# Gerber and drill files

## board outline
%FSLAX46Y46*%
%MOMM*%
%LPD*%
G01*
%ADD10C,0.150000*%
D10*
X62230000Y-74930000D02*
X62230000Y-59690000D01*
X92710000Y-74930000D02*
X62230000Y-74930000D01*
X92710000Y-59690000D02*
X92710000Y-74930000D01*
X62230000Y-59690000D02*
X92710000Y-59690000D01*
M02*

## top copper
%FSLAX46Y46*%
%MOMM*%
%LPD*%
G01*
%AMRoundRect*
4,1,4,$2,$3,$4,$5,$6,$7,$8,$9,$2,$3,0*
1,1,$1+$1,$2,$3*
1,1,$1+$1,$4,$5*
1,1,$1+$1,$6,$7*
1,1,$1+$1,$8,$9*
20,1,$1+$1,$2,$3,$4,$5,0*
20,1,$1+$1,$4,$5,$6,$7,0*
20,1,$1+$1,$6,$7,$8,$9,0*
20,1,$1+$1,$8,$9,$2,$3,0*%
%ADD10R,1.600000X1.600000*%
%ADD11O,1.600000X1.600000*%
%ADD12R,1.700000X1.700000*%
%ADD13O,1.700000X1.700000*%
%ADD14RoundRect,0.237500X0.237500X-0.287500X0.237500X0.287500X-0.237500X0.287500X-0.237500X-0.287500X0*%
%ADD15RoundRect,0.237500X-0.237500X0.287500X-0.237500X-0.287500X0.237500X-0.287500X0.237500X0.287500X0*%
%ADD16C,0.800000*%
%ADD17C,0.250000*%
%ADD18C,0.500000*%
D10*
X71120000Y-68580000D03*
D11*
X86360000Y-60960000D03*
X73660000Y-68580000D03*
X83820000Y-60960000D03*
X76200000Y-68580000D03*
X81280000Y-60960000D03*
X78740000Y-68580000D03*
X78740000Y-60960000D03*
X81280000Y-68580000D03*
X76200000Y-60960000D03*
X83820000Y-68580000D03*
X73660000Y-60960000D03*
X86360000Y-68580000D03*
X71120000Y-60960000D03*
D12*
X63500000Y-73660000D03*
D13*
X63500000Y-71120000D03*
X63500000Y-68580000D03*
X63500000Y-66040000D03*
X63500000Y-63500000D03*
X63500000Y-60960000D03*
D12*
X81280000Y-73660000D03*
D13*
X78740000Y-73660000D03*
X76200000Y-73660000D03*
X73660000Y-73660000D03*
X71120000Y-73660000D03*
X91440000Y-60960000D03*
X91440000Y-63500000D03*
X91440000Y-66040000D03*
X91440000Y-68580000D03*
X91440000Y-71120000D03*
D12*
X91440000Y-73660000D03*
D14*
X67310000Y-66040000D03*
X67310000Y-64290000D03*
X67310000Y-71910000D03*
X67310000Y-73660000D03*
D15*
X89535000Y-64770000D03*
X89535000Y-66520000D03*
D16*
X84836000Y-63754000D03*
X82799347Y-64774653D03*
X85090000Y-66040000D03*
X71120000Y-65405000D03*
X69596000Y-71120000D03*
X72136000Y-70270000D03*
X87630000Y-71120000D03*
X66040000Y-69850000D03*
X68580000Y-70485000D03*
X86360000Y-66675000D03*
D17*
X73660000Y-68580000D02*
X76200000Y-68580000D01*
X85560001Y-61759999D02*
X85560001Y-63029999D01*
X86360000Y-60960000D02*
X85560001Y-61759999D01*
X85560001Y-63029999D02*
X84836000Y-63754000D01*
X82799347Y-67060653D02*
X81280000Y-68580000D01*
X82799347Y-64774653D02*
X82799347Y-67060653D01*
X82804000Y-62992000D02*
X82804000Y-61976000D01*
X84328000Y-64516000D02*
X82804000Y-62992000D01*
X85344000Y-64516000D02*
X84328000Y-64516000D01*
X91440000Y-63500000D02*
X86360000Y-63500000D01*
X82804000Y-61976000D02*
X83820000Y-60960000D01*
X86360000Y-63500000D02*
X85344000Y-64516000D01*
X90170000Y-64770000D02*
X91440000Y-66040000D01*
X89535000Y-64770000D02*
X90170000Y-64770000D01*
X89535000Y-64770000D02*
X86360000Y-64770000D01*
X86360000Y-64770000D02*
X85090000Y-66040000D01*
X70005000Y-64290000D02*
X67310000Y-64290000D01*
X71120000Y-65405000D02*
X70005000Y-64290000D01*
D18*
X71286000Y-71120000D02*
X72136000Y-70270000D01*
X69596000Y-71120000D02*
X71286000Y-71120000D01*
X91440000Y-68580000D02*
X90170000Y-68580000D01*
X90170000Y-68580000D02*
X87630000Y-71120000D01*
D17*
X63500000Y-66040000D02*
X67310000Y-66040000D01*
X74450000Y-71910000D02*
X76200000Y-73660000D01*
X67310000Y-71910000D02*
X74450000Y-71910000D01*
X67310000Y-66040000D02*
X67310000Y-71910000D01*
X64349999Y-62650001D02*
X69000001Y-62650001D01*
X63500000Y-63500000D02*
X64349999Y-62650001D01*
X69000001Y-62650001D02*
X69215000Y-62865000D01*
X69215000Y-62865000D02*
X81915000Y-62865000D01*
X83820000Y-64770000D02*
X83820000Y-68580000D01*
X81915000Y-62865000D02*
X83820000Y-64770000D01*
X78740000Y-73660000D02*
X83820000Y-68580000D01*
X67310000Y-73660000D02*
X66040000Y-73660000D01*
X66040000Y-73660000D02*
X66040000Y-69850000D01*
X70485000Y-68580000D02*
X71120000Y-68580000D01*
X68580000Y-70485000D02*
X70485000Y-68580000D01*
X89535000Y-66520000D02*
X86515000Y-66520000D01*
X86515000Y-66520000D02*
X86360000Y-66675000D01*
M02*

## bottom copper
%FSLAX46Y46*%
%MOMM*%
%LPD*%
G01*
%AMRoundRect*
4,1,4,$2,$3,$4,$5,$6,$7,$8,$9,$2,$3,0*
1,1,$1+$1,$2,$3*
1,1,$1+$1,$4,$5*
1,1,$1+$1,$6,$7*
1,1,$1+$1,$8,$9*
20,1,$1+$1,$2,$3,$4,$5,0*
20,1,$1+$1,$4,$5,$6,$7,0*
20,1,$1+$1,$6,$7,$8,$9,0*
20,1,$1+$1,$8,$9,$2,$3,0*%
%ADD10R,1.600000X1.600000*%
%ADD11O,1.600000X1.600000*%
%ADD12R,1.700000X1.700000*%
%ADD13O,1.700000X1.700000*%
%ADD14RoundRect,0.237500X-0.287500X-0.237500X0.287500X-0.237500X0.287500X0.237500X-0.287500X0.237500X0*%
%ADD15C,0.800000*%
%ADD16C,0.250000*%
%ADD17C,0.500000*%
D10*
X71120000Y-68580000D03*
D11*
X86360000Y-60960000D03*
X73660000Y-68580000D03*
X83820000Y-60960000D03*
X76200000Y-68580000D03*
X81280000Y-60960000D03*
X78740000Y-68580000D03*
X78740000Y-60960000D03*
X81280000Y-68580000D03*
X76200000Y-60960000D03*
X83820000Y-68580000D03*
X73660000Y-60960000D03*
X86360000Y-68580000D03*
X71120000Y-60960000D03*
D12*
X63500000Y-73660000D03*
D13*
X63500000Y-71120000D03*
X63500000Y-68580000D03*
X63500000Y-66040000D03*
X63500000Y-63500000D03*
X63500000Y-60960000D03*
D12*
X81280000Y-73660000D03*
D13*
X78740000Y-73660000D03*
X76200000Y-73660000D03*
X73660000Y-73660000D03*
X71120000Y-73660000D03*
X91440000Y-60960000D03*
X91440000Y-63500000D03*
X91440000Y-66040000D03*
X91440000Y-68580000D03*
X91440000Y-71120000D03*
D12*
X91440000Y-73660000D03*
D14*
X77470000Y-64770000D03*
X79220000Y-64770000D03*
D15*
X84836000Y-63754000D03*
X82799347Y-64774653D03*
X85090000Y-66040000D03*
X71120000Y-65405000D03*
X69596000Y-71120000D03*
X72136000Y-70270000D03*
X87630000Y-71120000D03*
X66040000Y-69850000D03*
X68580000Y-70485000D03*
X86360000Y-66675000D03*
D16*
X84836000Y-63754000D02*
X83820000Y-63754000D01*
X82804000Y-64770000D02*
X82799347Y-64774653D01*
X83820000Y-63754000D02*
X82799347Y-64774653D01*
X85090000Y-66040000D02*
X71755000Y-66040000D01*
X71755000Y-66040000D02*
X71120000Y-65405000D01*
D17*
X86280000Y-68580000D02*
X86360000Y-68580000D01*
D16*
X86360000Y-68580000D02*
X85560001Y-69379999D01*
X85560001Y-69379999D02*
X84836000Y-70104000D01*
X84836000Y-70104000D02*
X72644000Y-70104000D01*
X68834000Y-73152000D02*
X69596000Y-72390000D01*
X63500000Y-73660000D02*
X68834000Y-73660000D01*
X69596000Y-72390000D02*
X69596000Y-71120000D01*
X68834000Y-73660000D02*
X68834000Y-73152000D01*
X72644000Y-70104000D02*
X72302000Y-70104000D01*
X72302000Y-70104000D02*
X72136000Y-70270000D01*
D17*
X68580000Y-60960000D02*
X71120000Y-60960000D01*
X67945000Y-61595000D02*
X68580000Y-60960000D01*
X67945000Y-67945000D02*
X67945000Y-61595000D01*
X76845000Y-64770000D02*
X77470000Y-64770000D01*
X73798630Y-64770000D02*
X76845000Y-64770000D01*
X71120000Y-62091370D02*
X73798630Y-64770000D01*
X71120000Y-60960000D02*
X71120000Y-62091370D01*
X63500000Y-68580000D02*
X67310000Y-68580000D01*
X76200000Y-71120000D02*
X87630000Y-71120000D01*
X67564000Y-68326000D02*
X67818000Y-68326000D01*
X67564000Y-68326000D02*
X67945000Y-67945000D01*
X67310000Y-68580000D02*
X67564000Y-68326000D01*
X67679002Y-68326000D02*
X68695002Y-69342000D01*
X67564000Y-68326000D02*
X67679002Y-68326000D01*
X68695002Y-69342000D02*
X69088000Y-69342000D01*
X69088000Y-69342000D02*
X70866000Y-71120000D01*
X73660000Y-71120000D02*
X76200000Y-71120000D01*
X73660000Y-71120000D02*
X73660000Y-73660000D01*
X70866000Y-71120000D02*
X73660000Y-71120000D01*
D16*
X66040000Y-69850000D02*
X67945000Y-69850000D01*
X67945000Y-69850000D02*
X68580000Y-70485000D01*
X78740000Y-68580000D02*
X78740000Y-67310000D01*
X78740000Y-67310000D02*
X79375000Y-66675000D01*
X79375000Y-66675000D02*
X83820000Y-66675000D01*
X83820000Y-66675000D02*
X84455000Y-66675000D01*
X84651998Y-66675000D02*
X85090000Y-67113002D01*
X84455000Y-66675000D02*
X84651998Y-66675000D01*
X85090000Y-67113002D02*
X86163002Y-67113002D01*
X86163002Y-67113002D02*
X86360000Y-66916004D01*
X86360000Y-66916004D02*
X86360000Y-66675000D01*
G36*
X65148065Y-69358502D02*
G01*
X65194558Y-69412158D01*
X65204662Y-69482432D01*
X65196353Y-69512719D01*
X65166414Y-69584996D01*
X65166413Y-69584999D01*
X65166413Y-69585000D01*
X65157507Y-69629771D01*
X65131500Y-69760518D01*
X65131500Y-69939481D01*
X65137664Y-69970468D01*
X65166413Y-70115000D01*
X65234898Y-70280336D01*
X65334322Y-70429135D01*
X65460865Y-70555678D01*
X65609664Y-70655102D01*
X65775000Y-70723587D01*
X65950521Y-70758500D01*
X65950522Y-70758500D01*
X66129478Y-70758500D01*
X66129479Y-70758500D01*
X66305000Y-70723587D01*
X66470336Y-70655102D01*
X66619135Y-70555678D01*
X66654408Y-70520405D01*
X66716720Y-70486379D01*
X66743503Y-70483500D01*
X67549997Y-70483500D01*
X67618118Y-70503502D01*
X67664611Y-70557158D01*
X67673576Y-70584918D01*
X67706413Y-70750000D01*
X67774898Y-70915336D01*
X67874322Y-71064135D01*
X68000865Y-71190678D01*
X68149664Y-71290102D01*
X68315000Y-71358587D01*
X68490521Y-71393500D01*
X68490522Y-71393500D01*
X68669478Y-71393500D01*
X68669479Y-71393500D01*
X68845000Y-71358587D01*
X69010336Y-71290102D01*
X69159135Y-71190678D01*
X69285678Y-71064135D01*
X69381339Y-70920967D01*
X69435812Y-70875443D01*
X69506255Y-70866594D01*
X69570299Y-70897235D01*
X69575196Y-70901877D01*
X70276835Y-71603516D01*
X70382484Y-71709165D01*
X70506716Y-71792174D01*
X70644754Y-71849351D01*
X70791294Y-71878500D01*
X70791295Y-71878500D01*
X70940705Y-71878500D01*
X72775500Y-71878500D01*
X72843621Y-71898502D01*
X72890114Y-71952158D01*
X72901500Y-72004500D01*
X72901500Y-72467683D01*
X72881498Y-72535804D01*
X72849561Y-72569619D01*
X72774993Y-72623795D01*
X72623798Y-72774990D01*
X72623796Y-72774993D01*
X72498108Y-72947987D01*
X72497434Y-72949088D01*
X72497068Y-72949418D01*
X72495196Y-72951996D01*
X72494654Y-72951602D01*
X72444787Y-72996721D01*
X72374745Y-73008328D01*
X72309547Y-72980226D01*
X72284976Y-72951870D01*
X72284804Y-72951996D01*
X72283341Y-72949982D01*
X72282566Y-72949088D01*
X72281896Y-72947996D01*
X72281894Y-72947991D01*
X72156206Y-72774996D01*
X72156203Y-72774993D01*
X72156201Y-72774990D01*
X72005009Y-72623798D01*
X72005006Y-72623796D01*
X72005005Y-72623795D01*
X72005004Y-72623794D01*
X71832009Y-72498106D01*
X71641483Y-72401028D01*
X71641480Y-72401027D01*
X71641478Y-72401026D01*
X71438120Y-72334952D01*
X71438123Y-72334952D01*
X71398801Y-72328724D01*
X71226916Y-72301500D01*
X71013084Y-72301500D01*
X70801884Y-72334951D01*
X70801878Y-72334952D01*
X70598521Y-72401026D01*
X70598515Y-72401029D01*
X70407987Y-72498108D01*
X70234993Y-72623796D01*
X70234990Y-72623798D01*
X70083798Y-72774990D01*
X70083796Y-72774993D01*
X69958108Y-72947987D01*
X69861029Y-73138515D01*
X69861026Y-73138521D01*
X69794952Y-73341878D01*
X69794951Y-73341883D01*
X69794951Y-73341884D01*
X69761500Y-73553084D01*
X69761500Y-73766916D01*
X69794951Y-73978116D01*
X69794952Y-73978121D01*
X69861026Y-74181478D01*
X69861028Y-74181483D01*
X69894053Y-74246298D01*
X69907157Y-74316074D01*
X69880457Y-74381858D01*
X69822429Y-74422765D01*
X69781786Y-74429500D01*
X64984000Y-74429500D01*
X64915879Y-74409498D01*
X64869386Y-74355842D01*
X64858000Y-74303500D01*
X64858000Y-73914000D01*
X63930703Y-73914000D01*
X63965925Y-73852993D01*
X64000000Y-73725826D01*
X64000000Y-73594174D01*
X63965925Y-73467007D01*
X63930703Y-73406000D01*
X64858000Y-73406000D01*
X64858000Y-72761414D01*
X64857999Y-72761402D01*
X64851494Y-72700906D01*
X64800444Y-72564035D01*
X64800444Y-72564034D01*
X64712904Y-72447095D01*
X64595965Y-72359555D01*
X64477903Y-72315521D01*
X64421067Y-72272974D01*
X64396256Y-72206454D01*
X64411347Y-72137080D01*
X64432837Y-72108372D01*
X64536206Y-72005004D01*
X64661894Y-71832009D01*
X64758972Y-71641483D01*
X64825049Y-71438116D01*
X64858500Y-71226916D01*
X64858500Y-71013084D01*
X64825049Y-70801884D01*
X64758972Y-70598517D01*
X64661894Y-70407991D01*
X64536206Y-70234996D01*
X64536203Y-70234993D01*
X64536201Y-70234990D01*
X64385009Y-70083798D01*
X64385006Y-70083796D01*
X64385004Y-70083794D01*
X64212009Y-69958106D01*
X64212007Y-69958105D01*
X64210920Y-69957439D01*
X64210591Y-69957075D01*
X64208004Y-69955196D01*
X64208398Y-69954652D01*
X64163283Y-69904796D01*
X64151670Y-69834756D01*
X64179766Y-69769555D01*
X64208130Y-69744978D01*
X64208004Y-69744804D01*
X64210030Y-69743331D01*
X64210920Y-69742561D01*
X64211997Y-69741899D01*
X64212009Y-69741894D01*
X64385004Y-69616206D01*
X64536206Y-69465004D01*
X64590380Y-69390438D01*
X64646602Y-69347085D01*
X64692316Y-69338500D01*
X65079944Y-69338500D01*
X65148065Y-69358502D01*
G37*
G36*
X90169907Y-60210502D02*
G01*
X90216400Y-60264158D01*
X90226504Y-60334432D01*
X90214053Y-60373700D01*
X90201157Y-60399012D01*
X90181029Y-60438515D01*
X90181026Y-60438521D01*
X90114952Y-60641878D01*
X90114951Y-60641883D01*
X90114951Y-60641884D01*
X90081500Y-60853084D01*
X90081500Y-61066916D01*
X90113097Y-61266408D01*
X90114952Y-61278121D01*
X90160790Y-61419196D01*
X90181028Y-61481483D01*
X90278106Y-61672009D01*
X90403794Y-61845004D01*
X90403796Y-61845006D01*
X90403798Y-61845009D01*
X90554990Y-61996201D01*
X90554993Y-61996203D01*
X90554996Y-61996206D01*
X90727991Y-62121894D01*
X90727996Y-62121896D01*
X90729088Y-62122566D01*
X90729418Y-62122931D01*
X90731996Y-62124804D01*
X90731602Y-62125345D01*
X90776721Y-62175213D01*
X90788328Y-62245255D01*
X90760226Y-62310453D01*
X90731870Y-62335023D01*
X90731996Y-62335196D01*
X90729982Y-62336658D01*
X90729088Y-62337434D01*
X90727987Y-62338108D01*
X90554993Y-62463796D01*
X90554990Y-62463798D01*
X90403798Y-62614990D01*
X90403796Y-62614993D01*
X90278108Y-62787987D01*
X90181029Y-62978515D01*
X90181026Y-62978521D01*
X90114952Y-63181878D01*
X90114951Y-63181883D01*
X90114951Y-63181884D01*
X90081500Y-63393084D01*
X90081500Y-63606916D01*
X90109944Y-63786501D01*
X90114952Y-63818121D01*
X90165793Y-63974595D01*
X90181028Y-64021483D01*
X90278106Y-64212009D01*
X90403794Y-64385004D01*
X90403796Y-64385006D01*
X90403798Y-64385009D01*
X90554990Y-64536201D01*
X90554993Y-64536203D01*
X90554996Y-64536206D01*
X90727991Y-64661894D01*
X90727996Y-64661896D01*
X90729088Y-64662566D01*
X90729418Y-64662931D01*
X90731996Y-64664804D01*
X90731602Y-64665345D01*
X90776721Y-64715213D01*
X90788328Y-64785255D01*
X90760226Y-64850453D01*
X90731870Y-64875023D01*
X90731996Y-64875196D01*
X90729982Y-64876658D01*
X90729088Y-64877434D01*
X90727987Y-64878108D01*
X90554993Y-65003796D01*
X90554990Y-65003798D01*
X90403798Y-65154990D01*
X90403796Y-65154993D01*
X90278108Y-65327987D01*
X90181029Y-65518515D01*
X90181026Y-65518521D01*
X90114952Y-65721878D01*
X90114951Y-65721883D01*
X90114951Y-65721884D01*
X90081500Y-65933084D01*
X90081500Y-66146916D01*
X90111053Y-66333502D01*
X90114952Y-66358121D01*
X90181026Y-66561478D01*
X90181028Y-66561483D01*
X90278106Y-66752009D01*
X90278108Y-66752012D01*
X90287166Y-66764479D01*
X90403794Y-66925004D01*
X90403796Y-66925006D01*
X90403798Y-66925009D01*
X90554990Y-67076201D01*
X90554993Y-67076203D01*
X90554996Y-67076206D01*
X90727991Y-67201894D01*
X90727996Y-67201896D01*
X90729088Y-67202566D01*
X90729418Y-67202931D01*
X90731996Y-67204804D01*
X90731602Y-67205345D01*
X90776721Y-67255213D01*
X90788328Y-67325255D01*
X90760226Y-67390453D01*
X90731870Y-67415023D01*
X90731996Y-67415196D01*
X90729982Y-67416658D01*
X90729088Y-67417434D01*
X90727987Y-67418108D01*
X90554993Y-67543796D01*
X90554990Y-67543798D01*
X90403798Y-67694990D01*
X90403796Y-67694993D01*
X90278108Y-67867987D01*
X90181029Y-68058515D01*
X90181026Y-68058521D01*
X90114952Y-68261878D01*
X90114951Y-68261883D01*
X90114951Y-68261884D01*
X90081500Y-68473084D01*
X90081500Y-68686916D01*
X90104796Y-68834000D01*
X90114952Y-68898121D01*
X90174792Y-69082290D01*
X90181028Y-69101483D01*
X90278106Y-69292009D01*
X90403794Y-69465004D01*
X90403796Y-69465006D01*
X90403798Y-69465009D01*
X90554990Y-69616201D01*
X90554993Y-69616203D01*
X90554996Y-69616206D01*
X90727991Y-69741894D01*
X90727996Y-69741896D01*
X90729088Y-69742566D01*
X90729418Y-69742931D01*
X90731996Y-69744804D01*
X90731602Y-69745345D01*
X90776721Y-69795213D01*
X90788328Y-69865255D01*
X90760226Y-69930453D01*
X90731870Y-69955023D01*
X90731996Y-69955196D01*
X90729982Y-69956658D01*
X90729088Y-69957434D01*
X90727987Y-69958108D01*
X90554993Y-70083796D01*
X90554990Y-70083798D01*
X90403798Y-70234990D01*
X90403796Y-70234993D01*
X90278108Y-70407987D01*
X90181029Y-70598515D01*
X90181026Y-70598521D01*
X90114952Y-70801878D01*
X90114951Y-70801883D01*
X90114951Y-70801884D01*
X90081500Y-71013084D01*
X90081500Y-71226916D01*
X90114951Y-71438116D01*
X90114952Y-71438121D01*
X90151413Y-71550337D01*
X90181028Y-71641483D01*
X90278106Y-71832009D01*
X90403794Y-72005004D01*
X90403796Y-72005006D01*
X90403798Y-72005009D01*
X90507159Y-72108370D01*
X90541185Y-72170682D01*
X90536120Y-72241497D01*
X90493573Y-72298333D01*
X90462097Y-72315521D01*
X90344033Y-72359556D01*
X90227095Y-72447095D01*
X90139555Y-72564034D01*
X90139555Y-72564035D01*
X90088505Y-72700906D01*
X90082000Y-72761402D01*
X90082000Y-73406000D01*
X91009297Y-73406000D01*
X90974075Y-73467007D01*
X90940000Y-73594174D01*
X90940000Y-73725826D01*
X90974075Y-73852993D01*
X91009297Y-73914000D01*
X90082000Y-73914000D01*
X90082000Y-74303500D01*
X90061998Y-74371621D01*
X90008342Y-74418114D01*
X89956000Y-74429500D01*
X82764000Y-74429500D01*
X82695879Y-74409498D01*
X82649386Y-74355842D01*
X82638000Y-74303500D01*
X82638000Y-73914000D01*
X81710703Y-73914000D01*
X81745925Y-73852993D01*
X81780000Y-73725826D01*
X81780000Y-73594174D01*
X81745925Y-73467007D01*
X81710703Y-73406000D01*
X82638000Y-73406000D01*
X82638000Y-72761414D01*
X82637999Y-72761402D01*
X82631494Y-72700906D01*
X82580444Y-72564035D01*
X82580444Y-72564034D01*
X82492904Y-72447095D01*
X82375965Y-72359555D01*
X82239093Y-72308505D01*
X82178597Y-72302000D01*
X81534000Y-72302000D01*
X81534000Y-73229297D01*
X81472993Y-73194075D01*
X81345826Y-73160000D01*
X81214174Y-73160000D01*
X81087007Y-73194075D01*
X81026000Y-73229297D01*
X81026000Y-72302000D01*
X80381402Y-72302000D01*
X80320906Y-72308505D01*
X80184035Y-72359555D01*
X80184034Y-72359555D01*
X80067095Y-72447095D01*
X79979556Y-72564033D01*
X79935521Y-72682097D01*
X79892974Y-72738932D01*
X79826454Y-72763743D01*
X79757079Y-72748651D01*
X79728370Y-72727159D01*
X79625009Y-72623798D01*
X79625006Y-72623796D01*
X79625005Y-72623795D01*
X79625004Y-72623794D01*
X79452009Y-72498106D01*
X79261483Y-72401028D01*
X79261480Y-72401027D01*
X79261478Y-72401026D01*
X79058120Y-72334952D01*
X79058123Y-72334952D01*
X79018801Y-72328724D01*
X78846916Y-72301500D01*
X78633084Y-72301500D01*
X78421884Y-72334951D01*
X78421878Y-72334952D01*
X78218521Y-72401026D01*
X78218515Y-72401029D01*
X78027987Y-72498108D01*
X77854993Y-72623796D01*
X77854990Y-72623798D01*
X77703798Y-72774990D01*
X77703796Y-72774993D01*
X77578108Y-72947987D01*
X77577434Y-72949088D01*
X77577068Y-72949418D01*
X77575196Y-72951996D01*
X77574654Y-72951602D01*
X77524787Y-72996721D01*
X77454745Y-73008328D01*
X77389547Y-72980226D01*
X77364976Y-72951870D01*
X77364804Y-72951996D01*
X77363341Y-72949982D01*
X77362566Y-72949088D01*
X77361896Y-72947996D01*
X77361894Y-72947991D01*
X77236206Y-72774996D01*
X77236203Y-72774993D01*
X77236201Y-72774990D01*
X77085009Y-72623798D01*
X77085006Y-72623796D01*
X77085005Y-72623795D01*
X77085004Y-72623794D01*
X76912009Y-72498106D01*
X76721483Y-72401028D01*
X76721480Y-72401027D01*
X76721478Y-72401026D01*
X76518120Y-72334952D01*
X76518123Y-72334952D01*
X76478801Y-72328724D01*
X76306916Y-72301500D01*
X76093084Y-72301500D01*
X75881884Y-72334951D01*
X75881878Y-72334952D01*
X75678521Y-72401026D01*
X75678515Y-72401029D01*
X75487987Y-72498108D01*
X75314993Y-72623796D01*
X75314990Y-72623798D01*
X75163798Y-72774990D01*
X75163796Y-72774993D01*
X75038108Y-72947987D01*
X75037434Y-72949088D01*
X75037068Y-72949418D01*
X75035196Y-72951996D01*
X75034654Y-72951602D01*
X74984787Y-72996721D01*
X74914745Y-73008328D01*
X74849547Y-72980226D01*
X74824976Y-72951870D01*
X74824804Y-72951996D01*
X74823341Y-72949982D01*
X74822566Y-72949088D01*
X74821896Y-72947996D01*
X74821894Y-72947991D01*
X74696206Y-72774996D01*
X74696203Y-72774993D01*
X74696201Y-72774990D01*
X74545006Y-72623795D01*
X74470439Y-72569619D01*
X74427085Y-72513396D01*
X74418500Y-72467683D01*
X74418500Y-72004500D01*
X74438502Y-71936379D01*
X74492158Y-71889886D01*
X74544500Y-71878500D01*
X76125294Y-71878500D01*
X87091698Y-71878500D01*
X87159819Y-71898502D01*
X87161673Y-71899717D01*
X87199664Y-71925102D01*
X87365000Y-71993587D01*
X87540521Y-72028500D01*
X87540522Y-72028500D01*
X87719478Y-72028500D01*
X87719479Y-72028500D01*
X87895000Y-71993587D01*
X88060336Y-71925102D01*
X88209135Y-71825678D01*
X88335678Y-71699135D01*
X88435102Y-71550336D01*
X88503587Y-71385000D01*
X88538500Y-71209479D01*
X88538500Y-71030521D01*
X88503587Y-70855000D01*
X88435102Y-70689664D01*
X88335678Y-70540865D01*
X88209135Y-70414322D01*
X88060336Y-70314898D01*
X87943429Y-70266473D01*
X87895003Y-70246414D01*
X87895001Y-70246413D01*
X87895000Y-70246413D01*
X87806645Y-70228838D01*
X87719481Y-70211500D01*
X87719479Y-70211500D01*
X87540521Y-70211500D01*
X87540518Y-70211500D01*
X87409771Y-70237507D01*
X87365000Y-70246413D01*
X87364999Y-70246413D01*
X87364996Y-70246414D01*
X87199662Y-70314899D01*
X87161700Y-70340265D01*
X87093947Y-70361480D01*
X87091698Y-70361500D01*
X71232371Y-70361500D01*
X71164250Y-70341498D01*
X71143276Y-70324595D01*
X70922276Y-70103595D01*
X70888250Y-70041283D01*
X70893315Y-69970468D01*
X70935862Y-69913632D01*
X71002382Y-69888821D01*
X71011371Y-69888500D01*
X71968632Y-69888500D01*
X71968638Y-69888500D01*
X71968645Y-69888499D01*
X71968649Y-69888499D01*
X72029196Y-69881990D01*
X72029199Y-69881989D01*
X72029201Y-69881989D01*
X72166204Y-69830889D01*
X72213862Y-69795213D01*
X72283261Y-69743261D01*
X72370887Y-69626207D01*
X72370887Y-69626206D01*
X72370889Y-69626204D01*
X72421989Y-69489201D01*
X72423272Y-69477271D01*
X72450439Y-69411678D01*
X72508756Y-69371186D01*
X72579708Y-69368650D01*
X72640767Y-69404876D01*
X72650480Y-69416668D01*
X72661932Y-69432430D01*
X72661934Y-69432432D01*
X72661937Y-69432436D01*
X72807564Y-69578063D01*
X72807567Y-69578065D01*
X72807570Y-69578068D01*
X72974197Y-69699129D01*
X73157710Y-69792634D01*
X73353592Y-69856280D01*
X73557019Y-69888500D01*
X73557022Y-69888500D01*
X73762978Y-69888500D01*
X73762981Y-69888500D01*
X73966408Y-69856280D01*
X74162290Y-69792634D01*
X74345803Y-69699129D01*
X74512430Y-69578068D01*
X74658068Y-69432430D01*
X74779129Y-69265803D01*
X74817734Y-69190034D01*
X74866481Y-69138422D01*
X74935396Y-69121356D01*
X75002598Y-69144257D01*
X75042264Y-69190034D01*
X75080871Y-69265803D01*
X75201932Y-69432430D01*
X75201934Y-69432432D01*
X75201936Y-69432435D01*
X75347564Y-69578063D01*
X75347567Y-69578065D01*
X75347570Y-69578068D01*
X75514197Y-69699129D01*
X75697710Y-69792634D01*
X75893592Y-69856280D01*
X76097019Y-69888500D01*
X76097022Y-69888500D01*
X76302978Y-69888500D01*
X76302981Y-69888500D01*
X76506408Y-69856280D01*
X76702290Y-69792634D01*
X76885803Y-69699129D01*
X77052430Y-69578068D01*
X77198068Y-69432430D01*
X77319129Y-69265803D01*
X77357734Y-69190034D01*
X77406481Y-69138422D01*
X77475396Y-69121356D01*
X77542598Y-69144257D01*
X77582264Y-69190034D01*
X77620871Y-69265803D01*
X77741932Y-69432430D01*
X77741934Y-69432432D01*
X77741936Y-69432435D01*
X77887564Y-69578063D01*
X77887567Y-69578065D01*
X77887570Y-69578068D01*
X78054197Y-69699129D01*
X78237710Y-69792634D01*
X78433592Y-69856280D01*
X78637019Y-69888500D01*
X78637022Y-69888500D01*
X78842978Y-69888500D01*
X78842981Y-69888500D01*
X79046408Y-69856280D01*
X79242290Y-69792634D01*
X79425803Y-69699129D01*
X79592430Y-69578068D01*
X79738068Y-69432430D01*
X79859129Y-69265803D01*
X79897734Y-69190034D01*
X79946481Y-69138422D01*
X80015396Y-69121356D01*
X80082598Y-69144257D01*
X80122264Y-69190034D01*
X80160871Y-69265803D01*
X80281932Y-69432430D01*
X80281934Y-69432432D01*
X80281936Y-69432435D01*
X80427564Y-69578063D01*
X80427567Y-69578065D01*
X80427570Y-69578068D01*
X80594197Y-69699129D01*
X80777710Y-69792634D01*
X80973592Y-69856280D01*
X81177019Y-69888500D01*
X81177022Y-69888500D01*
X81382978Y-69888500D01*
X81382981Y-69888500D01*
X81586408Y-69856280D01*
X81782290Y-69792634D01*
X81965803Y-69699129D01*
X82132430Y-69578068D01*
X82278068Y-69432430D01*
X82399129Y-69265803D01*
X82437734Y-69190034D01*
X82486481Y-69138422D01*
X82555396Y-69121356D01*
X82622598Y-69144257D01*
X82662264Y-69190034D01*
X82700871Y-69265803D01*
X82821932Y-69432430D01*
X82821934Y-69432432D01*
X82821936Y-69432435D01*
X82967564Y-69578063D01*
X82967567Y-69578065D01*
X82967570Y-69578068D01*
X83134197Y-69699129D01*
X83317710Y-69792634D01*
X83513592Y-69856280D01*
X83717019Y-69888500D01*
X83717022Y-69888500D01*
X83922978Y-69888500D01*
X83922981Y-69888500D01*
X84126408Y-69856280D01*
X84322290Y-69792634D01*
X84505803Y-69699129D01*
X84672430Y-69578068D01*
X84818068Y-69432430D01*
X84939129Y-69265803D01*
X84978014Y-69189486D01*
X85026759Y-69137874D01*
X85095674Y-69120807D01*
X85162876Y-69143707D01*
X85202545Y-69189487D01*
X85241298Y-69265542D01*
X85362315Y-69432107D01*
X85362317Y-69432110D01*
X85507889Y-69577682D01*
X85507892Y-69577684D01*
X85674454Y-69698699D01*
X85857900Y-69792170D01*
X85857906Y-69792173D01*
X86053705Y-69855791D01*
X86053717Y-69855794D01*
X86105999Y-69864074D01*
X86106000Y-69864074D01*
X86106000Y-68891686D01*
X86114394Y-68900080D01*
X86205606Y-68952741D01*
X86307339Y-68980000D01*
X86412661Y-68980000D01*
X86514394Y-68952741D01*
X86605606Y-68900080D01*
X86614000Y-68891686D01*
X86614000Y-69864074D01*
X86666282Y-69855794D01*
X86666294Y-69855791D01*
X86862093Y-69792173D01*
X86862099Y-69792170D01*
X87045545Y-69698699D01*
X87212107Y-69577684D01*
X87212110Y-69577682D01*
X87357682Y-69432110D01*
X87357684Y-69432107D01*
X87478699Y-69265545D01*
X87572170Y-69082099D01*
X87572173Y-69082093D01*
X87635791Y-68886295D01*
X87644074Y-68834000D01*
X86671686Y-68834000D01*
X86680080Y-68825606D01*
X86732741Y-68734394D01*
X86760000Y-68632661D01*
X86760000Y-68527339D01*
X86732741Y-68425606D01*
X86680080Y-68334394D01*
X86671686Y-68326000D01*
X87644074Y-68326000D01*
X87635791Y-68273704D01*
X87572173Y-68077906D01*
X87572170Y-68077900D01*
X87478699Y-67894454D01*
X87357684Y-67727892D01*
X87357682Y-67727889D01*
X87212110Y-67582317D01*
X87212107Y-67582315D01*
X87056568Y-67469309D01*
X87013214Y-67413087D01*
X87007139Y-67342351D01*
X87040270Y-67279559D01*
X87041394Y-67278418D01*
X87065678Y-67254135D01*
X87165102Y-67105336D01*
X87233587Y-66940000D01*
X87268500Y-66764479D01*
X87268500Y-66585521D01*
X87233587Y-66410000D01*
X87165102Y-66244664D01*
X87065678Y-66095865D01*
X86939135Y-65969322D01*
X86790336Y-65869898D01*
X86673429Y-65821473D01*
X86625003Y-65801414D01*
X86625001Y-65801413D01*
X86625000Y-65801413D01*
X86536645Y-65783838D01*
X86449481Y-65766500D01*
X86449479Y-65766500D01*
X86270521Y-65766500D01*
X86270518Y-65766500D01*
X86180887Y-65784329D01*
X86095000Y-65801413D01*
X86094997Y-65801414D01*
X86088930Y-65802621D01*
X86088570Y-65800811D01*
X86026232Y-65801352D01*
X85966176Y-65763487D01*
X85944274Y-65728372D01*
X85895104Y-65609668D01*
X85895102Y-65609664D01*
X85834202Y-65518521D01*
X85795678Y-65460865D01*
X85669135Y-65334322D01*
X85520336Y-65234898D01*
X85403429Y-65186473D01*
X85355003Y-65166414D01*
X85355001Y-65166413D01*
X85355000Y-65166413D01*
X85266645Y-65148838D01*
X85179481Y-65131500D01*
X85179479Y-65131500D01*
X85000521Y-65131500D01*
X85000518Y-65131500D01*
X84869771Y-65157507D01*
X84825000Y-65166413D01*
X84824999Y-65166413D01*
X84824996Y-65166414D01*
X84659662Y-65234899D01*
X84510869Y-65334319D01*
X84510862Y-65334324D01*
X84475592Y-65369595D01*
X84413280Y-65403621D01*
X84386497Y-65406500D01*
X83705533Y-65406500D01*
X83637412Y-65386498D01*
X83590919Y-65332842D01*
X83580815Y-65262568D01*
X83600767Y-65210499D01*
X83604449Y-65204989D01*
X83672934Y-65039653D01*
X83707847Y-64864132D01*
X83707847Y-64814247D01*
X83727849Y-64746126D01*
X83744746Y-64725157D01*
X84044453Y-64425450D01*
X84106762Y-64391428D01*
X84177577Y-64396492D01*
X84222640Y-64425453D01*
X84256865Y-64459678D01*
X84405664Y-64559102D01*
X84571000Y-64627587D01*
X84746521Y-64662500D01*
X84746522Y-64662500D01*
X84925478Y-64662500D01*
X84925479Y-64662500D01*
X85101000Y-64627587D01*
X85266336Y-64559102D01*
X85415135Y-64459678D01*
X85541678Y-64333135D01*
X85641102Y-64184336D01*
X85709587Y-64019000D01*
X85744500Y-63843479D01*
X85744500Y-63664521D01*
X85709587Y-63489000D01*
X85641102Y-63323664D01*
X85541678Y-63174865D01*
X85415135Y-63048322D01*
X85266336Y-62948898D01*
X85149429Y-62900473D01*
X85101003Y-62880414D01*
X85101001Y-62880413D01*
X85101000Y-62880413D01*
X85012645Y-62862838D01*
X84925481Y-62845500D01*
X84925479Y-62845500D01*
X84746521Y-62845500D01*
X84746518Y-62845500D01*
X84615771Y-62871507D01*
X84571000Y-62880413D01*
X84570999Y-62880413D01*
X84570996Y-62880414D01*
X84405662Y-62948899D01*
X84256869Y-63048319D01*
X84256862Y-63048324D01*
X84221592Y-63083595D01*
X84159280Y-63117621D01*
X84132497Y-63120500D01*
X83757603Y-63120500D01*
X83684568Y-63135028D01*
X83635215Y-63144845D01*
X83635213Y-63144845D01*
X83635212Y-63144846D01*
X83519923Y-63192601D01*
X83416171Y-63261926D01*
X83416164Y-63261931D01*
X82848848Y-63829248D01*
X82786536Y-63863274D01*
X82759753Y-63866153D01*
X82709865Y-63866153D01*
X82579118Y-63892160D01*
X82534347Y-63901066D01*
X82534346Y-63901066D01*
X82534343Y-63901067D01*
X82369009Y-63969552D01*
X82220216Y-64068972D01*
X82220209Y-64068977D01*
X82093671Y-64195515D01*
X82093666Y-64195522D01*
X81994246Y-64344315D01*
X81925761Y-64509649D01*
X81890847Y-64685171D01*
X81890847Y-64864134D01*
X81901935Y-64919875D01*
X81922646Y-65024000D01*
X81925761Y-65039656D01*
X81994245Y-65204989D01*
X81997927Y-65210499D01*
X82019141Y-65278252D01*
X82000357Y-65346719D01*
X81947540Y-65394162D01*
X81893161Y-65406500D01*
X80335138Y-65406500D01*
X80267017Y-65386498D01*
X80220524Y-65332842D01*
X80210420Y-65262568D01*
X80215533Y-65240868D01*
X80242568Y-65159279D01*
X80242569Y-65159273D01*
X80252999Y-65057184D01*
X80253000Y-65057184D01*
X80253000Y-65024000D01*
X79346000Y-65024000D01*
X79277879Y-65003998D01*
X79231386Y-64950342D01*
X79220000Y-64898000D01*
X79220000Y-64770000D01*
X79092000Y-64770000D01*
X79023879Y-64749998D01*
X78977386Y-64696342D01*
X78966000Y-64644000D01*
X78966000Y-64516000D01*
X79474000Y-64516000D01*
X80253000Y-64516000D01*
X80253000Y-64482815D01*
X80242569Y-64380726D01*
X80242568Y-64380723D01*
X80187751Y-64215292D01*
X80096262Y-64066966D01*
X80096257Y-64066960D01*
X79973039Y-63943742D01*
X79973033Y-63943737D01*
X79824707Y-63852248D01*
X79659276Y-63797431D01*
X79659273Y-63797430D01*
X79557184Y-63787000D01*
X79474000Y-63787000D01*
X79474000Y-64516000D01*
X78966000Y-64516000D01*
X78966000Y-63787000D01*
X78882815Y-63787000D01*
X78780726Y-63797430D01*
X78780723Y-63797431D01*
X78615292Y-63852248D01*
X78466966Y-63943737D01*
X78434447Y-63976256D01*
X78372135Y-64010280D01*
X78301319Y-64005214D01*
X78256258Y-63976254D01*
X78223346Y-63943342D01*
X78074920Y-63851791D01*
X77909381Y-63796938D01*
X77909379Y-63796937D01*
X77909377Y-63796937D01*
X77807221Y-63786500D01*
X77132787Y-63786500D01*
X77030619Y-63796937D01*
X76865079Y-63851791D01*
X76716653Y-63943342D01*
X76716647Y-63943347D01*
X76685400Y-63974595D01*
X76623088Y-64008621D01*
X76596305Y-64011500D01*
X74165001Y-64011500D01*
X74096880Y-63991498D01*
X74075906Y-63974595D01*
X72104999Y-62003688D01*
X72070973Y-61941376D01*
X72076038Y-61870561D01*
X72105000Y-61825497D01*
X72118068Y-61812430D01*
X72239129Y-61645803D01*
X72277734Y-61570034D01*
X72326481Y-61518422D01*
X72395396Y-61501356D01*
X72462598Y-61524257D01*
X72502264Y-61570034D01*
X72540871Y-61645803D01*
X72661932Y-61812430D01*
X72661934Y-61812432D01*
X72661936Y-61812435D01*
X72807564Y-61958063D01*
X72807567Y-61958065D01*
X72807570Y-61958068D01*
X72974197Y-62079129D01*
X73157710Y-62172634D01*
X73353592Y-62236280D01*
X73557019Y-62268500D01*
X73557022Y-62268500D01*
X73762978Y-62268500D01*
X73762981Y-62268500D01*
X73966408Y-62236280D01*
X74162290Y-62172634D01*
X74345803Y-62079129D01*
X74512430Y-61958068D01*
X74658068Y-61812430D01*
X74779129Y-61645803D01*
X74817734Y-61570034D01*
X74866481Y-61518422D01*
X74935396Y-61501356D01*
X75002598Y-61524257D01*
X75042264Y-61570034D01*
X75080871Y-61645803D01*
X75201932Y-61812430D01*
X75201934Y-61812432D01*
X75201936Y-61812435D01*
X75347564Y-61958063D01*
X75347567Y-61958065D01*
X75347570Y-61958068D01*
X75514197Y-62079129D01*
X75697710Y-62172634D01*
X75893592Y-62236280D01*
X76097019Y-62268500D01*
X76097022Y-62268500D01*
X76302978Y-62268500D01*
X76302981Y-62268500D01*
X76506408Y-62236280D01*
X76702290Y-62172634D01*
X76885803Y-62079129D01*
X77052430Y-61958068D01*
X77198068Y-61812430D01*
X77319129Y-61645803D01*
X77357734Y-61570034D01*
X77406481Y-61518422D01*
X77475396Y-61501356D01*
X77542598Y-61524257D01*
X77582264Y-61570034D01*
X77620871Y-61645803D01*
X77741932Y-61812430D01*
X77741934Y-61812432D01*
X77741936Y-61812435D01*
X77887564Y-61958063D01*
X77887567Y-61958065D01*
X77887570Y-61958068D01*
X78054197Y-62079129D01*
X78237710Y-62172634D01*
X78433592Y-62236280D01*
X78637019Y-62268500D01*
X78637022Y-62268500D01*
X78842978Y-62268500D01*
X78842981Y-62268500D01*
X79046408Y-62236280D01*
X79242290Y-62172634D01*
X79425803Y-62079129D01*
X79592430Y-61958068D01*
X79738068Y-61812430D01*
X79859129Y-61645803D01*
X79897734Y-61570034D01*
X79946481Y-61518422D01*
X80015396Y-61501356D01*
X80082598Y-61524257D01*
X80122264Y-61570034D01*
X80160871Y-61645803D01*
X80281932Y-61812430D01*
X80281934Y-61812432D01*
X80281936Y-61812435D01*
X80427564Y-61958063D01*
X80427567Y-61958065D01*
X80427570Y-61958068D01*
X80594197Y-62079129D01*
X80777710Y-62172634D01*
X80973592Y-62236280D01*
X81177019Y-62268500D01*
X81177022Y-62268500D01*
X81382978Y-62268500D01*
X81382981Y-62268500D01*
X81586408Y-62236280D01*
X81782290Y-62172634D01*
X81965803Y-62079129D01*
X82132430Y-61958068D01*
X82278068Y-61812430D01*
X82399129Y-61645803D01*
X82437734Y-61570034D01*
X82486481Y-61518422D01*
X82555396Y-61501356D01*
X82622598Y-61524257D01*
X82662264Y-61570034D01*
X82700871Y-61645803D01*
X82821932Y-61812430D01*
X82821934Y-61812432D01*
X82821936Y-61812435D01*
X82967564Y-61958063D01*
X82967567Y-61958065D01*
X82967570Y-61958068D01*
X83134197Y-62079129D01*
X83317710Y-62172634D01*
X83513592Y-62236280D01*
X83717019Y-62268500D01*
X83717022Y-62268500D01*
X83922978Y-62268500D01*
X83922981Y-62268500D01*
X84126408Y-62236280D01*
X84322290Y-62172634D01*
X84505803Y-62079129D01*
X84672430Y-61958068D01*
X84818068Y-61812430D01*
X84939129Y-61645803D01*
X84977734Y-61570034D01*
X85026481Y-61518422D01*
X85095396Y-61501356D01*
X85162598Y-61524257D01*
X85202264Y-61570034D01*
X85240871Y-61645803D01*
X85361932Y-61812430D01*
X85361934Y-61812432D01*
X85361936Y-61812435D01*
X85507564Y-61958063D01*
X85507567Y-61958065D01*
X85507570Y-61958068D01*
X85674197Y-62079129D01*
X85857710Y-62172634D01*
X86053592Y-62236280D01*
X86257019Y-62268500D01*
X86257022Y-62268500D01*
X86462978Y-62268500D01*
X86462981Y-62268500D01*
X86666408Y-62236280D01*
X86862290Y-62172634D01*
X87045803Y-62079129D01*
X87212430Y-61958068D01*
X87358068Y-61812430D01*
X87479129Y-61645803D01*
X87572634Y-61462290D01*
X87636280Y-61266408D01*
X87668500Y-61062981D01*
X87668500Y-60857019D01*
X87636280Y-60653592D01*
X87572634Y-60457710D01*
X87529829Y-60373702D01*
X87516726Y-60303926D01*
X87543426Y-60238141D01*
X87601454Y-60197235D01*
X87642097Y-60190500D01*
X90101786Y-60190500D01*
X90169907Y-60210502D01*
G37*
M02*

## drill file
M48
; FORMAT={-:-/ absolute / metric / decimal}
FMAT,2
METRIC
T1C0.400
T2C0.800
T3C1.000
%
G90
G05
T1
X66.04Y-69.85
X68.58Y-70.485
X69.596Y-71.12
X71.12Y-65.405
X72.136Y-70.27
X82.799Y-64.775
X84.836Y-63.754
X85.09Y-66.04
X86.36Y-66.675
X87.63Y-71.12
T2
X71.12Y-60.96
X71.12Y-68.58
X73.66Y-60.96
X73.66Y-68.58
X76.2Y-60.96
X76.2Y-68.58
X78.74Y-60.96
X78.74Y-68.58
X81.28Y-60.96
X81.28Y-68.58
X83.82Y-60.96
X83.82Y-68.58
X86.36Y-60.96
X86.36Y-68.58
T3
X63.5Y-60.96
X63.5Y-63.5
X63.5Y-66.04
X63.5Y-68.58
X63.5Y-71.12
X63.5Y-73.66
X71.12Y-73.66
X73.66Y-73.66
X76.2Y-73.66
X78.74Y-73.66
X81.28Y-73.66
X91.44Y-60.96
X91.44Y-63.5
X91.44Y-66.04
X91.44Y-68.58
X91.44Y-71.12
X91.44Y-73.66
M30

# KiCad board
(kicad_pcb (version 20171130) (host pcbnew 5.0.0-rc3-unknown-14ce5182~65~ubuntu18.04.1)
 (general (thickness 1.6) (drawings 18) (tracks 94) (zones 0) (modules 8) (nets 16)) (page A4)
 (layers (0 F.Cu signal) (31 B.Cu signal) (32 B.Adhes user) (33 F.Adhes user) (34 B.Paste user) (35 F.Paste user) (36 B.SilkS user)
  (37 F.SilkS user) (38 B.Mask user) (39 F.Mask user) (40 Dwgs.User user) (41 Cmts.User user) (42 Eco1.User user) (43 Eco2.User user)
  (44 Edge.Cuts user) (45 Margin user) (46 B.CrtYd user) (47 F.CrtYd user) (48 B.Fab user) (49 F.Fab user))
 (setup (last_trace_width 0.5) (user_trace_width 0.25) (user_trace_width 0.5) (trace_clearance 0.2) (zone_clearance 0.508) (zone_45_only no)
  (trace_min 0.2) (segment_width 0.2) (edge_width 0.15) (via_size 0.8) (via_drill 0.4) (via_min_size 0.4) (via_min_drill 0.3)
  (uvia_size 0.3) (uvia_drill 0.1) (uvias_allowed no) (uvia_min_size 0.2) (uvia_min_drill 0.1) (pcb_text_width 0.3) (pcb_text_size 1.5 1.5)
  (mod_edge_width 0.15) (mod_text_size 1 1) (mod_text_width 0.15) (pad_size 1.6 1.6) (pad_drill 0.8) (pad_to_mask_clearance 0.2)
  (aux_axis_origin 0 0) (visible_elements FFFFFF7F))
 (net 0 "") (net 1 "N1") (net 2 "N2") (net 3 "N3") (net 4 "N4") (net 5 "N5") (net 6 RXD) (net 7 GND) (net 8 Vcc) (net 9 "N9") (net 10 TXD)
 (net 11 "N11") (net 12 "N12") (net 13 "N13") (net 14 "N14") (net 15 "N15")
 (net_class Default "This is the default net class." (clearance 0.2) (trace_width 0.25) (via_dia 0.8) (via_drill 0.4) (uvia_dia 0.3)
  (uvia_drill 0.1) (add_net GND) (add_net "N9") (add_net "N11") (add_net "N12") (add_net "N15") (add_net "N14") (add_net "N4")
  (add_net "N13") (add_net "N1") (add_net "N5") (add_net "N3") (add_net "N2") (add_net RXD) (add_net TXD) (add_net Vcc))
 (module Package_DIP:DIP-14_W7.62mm (layer F.Cu) (at 71.12 68.58 90)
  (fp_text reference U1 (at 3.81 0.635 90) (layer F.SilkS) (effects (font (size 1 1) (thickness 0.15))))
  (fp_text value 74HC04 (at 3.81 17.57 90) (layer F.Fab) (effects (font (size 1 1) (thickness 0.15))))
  (pad 1 thru_hole rect (at 0 0 90) (size 1.6 1.6) (drill 0.8) (layers *.Cu *.Mask) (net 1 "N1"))
  (pad 8 thru_hole oval (at 7.62 15.24 90) (size 1.6 1.6) (drill 0.8) (layers *.Cu *.Mask) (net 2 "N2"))
  (pad 2 thru_hole oval (at 0 2.54 90) (size 1.6 1.6) (drill 0.8) (layers *.Cu *.Mask) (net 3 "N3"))
  (pad 9 thru_hole oval (at 7.62 12.7 90) (size 1.6 1.6) (drill 0.8) (layers *.Cu *.Mask) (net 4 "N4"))
  (pad 3 thru_hole oval (at 0 5.08 90) (size 1.6 1.6) (drill 0.8) (layers *.Cu *.Mask) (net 3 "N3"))
  (pad 10 thru_hole oval (at 7.62 10.16 90) (size 1.6 1.6) (drill 0.8) (layers *.Cu *.Mask))
  (pad 4 thru_hole oval (at 0 7.62 90) (size 1.6 1.6) (drill 0.8) (layers *.Cu *.Mask) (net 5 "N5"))
  (pad 11 thru_hole oval (at 7.62 7.62 90) (size 1.6 1.6) (drill 0.8) (layers *.Cu *.Mask))
  (pad 5 thru_hole oval (at 0 10.16 90) (size 1.6 1.6) (drill 0.8) (layers *.Cu *.Mask) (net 2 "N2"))
  (pad 12 thru_hole oval (at 7.62 5.08 90) (size 1.6 1.6) (drill 0.8) (layers *.Cu *.Mask))
  (pad 6 thru_hole oval (at 0 12.7 90) (size 1.6 1.6) (drill 0.8) (layers *.Cu *.Mask) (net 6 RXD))
  (pad 13 thru_hole oval (at 7.62 2.54 90) (size 1.6 1.6) (drill 0.8) (layers *.Cu *.Mask))
  (pad 7 thru_hole oval (at 0 15.24 90) (size 1.6 1.6) (drill 0.8) (layers *.Cu *.Mask) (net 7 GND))
  (pad 14 thru_hole oval (at 7.62 0 90) (size 1.6 1.6) (drill 0.8) (layers *.Cu *.Mask) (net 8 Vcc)))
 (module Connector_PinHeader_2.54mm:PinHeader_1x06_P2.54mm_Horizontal (layer F.Cu) (at 63.5 73.66 180)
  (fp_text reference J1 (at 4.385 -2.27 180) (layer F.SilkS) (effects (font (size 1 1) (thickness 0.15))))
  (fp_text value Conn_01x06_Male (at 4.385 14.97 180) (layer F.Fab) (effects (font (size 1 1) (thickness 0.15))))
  (pad 1 thru_hole rect (at 0 0 180) (size 1.7 1.7) (drill 1) (layers *.Cu *.Mask) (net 7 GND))
  (pad 2 thru_hole oval (at 0 2.54 180) (size 1.7 1.7) (drill 1) (layers *.Cu *.Mask) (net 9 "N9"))
  (pad 3 thru_hole oval (at 0 5.08 180) (size 1.7 1.7) (drill 1) (layers *.Cu *.Mask) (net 8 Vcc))
  (pad 4 thru_hole oval (at 0 7.62 180) (size 1.7 1.7) (drill 1) (layers *.Cu *.Mask) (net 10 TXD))
  (pad 5 thru_hole oval (at 0 10.16 180) (size 1.7 1.7) (drill 1) (layers *.Cu *.Mask) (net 6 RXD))
  (pad 6 thru_hole oval (at 0 12.7 180) (size 1.7 1.7) (drill 1) (layers *.Cu *.Mask) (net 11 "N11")))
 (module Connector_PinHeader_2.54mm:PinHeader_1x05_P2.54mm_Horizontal (layer F.Cu) (at 81.28 73.66 270)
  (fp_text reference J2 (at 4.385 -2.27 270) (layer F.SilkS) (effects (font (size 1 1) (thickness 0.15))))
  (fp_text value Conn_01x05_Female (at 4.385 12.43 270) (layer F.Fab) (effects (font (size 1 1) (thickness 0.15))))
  (pad 1 thru_hole rect (at 0 0 270) (size 1.7 1.7) (drill 1) (layers *.Cu *.Mask) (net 7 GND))
  (pad 2 thru_hole oval (at 0 2.54 270) (size 1.7 1.7) (drill 1) (layers *.Cu *.Mask) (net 6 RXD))
  (pad 3 thru_hole oval (at 0 5.08 270) (size 1.7 1.7) (drill 1) (layers *.Cu *.Mask) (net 10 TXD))
  (pad 4 thru_hole oval (at 0 7.62 270) (size 1.7 1.7) (drill 1) (layers *.Cu *.Mask) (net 8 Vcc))
  (pad 5 thru_hole oval (at 0 10.16 270) (size 1.7 1.7) (drill 1) (layers *.Cu *.Mask) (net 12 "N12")))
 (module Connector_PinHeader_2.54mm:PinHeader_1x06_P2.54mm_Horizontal (layer B.Cu) (at 91.44 73.66)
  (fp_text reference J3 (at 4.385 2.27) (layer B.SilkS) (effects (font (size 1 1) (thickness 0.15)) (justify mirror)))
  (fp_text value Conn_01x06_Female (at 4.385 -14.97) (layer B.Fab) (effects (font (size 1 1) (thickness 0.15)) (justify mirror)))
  (pad 6 thru_hole oval (at 0 -12.7) (size 1.7 1.7) (drill 1) (layers *.Cu *.Mask) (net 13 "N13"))
  (pad 5 thru_hole oval (at 0 -10.16) (size 1.7 1.7) (drill 1) (layers *.Cu *.Mask) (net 4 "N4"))
  (pad 4 thru_hole oval (at 0 -7.62) (size 1.7 1.7) (drill 1) (layers *.Cu *.Mask) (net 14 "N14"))
  (pad 3 thru_hole oval (at 0 -5.08) (size 1.7 1.7) (drill 1) (layers *.Cu *.Mask) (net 8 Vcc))
  (pad 2 thru_hole oval (at 0 -2.54) (size 1.7 1.7) (drill 1) (layers *.Cu *.Mask) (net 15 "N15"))
  (pad 1 thru_hole rect (at 0 0) (size 1.7 1.7) (drill 1) (layers *.Cu *.Mask) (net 7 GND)))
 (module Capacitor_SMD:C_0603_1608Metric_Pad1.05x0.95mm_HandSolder (layer B.Cu) (at 78.345 64.77)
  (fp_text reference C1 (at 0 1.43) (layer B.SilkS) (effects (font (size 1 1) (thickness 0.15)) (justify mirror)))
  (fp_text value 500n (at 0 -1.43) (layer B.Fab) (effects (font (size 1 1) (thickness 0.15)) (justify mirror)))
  (pad 1 smd roundrect (at -0.875 0) (size 1.05 0.95) (layers B.Cu B.Paste B.Mask) (roundrect_rratio 0.25) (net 8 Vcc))
  (pad 2 smd roundrect (at 0.875 0) (size 1.05 0.95) (layers B.Cu B.Paste B.Mask) (roundrect_rratio 0.25) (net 7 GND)))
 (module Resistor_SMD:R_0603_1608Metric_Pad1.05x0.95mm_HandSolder (layer F.Cu) (at 67.31 65.165 90)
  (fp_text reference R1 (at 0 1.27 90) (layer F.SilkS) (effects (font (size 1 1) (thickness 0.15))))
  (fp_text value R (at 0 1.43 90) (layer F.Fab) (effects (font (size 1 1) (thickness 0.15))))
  (pad 1 smd roundrect (at -0.875 0 90) (size 1.05 0.95) (layers F.Cu F.Paste F.Mask) (roundrect_rratio 0.25) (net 10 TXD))
  (pad 2 smd roundrect (at 0.875 0 90) (size 1.05 0.95) (layers F.Cu F.Paste F.Mask) (roundrect_rratio 0.25) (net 14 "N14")))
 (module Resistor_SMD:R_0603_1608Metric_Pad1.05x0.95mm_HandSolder (layer F.Cu) (at 67.31 72.785 90)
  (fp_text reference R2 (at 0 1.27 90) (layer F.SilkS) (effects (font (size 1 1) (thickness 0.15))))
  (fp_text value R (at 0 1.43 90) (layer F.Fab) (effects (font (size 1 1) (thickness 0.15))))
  (pad 2 smd roundrect (at 0.875 0 90) (size 1.05 0.95) (layers F.Cu F.Paste F.Mask) (roundrect_rratio 0.25) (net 10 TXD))
  (pad 1 smd roundrect (at -0.875 0 90) (size 1.05 0.95) (layers F.Cu F.Paste F.Mask) (roundrect_rratio 0.25) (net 1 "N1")))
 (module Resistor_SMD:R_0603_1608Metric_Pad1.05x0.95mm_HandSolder (layer F.Cu) (at 89.535 65.645 270)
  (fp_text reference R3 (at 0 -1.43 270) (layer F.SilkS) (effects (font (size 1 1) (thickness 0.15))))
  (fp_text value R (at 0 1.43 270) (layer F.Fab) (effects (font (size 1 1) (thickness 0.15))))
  (pad 1 smd roundrect (at -0.875 0 270) (size 1.05 0.95) (layers F.Cu F.Paste F.Mask) (roundrect_rratio 0.25) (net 14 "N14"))
  (pad 2 smd roundrect (at 0.875 0 270) (size 1.05 0.95) (layers F.Cu F.Paste F.Mask) (roundrect_rratio 0.25) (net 5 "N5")))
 (gr_line (start 62.23 74.93) (end 62.23 59.69) (layer Edge.Cuts) (width 0.15))
 (gr_line (start 92.71 74.93) (end 62.23 74.93) (layer Edge.Cuts) (width 0.15))
 (gr_line (start 92.71 59.69) (end 92.71 74.93) (layer Edge.Cuts) (width 0.15))
 (gr_line (start 62.23 59.69) (end 92.71 59.69) (layer Edge.Cuts) (width 0.15))
 (segment (start 73.66 68.58) (end 76.2 68.58) (width 0.25) (layer F.Cu) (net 3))
 (segment (start 85.560001 61.759999) (end 85.560001 63.029999) (width 0.25) (layer F.Cu) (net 2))
 (segment (start 86.36 60.96) (end 85.560001 61.759999) (width 0.25) (layer F.Cu) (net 2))
 (segment (start 85.560001 63.029999) (end 84.836 63.754) (width 0.25) (layer F.Cu) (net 2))
 (via (at 84.836 63.754) (size 0.8) (drill 0.4) (layers F.Cu B.Cu) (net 2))
 (segment (start 84.836 63.754) (end 83.82 63.754) (width 0.25) (layer B.Cu) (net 2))
 (via (at 82.799347 64.774653) (size 0.8) (drill 0.4) (layers F.Cu B.Cu) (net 2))
 (segment (start 82.804 64.77) (end 82.799347 64.774653) (width 0.25) (layer B.Cu) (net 2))
 (segment (start 83.82 63.754) (end 82.799347 64.774653) (width 0.25) (layer B.Cu) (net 2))
 (segment (start 82.799347 67.060653) (end 81.28 68.58) (width 0.25) (layer F.Cu) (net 2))
 (segment (start 82.799347 64.774653) (end 82.799347 67.060653) (width 0.25) (layer F.Cu) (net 2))
 (segment (start 82.804 62.992) (end 82.804 61.976) (width 0.25) (layer F.Cu) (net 4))
 (segment (start 84.328 64.516) (end 82.804 62.992) (width 0.25) (layer F.Cu) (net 4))
 (segment (start 85.344 64.516) (end 84.328 64.516) (width 0.25) (layer F.Cu) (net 4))
 (segment (start 91.44 63.5) (end 86.36 63.5) (width 0.25) (layer F.Cu) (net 4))
 (segment (start 82.804 61.976) (end 83.82 60.96) (width 0.25) (layer F.Cu) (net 4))
 (segment (start 86.36 63.5) (end 85.344 64.516) (width 0.25) (layer F.Cu) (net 4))
 (segment (start 90.17 64.77) (end 91.44 66.04) (width 0.25) (layer F.Cu) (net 14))
 (segment (start 89.535 64.77) (end 90.17 64.77) (width 0.25) (layer F.Cu) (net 14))
 (segment (start 89.535 64.77) (end 86.36 64.77) (width 0.25) (layer F.Cu) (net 14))
 (segment (start 86.36 64.77) (end 85.09 66.04) (width 0.25) (layer F.Cu) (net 14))
 (via (at 85.09 66.04) (size 0.8) (drill 0.4) (layers F.Cu B.Cu) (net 14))
 (via (at 71.12 65.405) (size 0.8) (drill 0.4) (layers F.Cu B.Cu) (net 14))
 (segment (start 85.09 66.04) (end 71.755 66.04) (width 0.25) (layer B.Cu) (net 14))
 (segment (start 71.755 66.04) (end 71.12 65.405) (width 0.25) (layer B.Cu) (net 14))
 (segment (start 70.005 64.29) (end 67.31 64.29) (width 0.25) (layer F.Cu) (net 14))
 (segment (start 71.12 65.405) (end 70.005 64.29) (width 0.25) (layer F.Cu) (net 14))
 (segment (start 86.28 68.58) (end 86.36 68.58) (width 0.5) (layer B.Cu) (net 7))
 (segment (start 86.36 68.58) (end 85.560001 69.379999) (width 0.25) (layer B.Cu) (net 7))
 (segment (start 85.560001 69.379999) (end 84.836 70.104) (width 0.25) (layer B.Cu) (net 7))
 (segment (start 84.836 70.104) (end 72.644 70.104) (width 0.25) (layer B.Cu) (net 7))
 (via (at 69.596 71.12) (size 0.8) (drill 0.4) (layers F.Cu B.Cu) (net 7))
 (segment (start 68.834 73.152) (end 69.596 72.39) (width 0.25) (layer B.Cu) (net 7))
 (segment (start 63.5 73.66) (end 68.834 73.66) (width 0.25) (layer B.Cu) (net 7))
 (segment (start 69.596 72.39) (end 69.596 71.12) (width 0.25) (layer B.Cu) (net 7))
 (segment (start 68.834 73.66) (end 68.834 73.152) (width 0.25) (layer B.Cu) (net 7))
 (via (at 72.136 70.27) (size 0.8) (drill 0.4) (layers F.Cu B.Cu) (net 7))
 (segment (start 72.644 70.104) (end 72.302 70.104) (width 0.25) (layer B.Cu) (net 7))
 (segment (start 72.302 70.104) (end 72.136 70.27) (width 0.25) (layer B.Cu) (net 7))
 (segment (start 71.286 71.12) (end 72.136 70.27) (width 0.5) (layer F.Cu) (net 7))
 (segment (start 69.596 71.12) (end 71.286 71.12) (width 0.5) (layer F.Cu) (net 7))
 (segment (start 68.58 60.96) (end 71.12 60.96) (width 0.5) (layer B.Cu) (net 8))
 (segment (start 67.945 61.595) (end 68.58 60.96) (width 0.5) (layer B.Cu) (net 8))
 (segment (start 67.945 67.945) (end 67.945 61.595) (width 0.5) (layer B.Cu) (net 8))
 (segment (start 76.845 64.77) (end 77.47 64.77) (width 0.5) (layer B.Cu) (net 8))
 (segment (start 73.79863 64.77) (end 76.845 64.77) (width 0.5) (layer B.Cu) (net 8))
 (segment (start 71.12 62.09137) (end 73.79863 64.77) (width 0.5) (layer B.Cu) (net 8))
 (segment (start 71.12 60.96) (end 71.12 62.09137) (width 0.5) (layer B.Cu) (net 8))
 (segment (start 63.5 68.58) (end 67.31 68.58) (width 0.5) (layer B.Cu) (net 8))
 (segment (start 91.44 68.58) (end 90.17 68.58) (width 0.5) (layer F.Cu) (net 8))
 (segment (start 90.17 68.58) (end 87.63 71.12) (width 0.5) (layer F.Cu) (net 8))
 (via (at 87.63 71.12) (size 0.8) (drill 0.4) (layers F.Cu B.Cu) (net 8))
 (segment (start 76.2 71.12) (end 87.63 71.12) (width 0.5) (layer B.Cu) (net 8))
 (segment (start 67.564 68.326) (end 67.818 68.326) (width 0.5) (layer B.Cu) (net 8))
 (segment (start 67.564 68.326) (end 67.945 67.945) (width 0.5) (layer B.Cu) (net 8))
 (segment (start 67.31 68.58) (end 67.564 68.326) (width 0.5) (layer B.Cu) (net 8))
 (segment (start 67.679002 68.326) (end 68.695002 69.342) (width 0.5) (layer B.Cu) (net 8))
 (segment (start 67.564 68.326) (end 67.679002 68.326) (width 0.5) (layer B.Cu) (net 8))
 (segment (start 68.695002 69.342) (end 69.088 69.342) (width 0.5) (layer B.Cu) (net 8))
 (segment (start 69.088 69.342) (end 70.866 71.12) (width 0.5) (layer B.Cu) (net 8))
 (segment (start 73.66 71.12) (end 76.2 71.12) (width 0.5) (layer B.Cu) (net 8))
 (segment (start 73.66 71.12) (end 73.66 73.66) (width 0.5) (layer B.Cu) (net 8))
 (segment (start 70.866 71.12) (end 73.66 71.12) (width 0.5) (layer B.Cu) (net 8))
 (segment (start 63.5 66.04) (end 67.31 66.04) (width 0.25) (layer F.Cu) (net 10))
 (segment (start 74.45 71.91) (end 76.2 73.66) (width 0.25) (layer F.Cu) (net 10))
 (segment (start 67.31 71.91) (end 74.45 71.91) (width 0.25) (layer F.Cu) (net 10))
 (segment (start 67.31 66.04) (end 67.31 71.91) (width 0.25) (layer F.Cu) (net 10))
 (segment (start 64.349999 62.650001) (end 69.000001 62.650001) (width 0.25) (layer F.Cu) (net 6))
 (segment (start 63.5 63.5) (end 64.349999 62.650001) (width 0.25) (layer F.Cu) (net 6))
 (segment (start 69.000001 62.650001) (end 69.215 62.865) (width 0.25) (layer F.Cu) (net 6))
 (segment (start 69.215 62.865) (end 81.915 62.865) (width 0.25) (layer F.Cu) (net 6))
 (segment (start 83.82 64.77) (end 83.82 68.58) (width 0.25) (layer F.Cu) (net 6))
 (segment (start 81.915 62.865) (end 83.82 64.77) (width 0.25) (layer F.Cu) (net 6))
 (segment (start 78.74 73.66) (end 83.82 68.58) (width 0.25) (layer F.Cu) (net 6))
 (segment (start 67.31 73.66) (end 66.04 73.66) (width 0.25) (layer F.Cu) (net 1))
 (via (at 66.04 69.85) (size 0.8) (drill 0.4) (layers F.Cu B.Cu) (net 1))
 (segment (start 66.04 73.66) (end 66.04 69.85) (width 0.25) (layer F.Cu) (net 1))
 (segment (start 66.04 69.85) (end 67.945 69.85) (width 0.25) (layer B.Cu) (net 1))
 (segment (start 67.945 69.85) (end 68.58 70.485) (width 0.25) (layer B.Cu) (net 1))
 (via (at 68.58 70.485) (size 0.8) (drill 0.4) (layers F.Cu B.Cu) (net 1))
 (segment (start 70.485 68.58) (end 71.12 68.58) (width 0.25) (layer F.Cu) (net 1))
 (segment (start 68.58 70.485) (end 70.485 68.58) (width 0.25) (layer F.Cu) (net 1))
 (segment (start 78.74 68.58) (end 78.74 67.31) (width 0.25) (layer B.Cu) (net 5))
 (segment (start 78.74 67.31) (end 79.375 66.675) (width 0.25) (layer B.Cu) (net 5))
 (segment (start 79.375 66.675) (end 83.82 66.675) (width 0.25) (layer B.Cu) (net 5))
 (segment (start 83.82 66.675) (end 84.455 66.675) (width 0.25) (layer B.Cu) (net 5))
 (segment (start 84.651998 66.675) (end 85.09 67.113002) (width 0.25) (layer B.Cu) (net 5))
 (segment (start 84.455 66.675) (end 84.651998 66.675) (width 0.25) (layer B.Cu) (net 5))
 (segment (start 85.09 67.113002) (end 86.163002 67.113002) (width 0.25) (layer B.Cu) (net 5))
 (segment (start 86.163002 67.113002) (end 86.36 66.916004) (width 0.25) (layer B.Cu) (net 5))
 (segment (start 86.36 66.916004) (end 86.36 66.675) (width 0.25) (layer B.Cu) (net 5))
 (via (at 86.36 66.675) (size 0.8) (drill 0.4) (layers F.Cu B.Cu) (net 5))
 (segment (start 89.535 66.52) (end 86.515 66.52) (width 0.25) (layer F.Cu) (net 5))
 (segment (start 86.515 66.52) (end 86.36 66.675) (width 0.25) (layer F.Cu) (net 5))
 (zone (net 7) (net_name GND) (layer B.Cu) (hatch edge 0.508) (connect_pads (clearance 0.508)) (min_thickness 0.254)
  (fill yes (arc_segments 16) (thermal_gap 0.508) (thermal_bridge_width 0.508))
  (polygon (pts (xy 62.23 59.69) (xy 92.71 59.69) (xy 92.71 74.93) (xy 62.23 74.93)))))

